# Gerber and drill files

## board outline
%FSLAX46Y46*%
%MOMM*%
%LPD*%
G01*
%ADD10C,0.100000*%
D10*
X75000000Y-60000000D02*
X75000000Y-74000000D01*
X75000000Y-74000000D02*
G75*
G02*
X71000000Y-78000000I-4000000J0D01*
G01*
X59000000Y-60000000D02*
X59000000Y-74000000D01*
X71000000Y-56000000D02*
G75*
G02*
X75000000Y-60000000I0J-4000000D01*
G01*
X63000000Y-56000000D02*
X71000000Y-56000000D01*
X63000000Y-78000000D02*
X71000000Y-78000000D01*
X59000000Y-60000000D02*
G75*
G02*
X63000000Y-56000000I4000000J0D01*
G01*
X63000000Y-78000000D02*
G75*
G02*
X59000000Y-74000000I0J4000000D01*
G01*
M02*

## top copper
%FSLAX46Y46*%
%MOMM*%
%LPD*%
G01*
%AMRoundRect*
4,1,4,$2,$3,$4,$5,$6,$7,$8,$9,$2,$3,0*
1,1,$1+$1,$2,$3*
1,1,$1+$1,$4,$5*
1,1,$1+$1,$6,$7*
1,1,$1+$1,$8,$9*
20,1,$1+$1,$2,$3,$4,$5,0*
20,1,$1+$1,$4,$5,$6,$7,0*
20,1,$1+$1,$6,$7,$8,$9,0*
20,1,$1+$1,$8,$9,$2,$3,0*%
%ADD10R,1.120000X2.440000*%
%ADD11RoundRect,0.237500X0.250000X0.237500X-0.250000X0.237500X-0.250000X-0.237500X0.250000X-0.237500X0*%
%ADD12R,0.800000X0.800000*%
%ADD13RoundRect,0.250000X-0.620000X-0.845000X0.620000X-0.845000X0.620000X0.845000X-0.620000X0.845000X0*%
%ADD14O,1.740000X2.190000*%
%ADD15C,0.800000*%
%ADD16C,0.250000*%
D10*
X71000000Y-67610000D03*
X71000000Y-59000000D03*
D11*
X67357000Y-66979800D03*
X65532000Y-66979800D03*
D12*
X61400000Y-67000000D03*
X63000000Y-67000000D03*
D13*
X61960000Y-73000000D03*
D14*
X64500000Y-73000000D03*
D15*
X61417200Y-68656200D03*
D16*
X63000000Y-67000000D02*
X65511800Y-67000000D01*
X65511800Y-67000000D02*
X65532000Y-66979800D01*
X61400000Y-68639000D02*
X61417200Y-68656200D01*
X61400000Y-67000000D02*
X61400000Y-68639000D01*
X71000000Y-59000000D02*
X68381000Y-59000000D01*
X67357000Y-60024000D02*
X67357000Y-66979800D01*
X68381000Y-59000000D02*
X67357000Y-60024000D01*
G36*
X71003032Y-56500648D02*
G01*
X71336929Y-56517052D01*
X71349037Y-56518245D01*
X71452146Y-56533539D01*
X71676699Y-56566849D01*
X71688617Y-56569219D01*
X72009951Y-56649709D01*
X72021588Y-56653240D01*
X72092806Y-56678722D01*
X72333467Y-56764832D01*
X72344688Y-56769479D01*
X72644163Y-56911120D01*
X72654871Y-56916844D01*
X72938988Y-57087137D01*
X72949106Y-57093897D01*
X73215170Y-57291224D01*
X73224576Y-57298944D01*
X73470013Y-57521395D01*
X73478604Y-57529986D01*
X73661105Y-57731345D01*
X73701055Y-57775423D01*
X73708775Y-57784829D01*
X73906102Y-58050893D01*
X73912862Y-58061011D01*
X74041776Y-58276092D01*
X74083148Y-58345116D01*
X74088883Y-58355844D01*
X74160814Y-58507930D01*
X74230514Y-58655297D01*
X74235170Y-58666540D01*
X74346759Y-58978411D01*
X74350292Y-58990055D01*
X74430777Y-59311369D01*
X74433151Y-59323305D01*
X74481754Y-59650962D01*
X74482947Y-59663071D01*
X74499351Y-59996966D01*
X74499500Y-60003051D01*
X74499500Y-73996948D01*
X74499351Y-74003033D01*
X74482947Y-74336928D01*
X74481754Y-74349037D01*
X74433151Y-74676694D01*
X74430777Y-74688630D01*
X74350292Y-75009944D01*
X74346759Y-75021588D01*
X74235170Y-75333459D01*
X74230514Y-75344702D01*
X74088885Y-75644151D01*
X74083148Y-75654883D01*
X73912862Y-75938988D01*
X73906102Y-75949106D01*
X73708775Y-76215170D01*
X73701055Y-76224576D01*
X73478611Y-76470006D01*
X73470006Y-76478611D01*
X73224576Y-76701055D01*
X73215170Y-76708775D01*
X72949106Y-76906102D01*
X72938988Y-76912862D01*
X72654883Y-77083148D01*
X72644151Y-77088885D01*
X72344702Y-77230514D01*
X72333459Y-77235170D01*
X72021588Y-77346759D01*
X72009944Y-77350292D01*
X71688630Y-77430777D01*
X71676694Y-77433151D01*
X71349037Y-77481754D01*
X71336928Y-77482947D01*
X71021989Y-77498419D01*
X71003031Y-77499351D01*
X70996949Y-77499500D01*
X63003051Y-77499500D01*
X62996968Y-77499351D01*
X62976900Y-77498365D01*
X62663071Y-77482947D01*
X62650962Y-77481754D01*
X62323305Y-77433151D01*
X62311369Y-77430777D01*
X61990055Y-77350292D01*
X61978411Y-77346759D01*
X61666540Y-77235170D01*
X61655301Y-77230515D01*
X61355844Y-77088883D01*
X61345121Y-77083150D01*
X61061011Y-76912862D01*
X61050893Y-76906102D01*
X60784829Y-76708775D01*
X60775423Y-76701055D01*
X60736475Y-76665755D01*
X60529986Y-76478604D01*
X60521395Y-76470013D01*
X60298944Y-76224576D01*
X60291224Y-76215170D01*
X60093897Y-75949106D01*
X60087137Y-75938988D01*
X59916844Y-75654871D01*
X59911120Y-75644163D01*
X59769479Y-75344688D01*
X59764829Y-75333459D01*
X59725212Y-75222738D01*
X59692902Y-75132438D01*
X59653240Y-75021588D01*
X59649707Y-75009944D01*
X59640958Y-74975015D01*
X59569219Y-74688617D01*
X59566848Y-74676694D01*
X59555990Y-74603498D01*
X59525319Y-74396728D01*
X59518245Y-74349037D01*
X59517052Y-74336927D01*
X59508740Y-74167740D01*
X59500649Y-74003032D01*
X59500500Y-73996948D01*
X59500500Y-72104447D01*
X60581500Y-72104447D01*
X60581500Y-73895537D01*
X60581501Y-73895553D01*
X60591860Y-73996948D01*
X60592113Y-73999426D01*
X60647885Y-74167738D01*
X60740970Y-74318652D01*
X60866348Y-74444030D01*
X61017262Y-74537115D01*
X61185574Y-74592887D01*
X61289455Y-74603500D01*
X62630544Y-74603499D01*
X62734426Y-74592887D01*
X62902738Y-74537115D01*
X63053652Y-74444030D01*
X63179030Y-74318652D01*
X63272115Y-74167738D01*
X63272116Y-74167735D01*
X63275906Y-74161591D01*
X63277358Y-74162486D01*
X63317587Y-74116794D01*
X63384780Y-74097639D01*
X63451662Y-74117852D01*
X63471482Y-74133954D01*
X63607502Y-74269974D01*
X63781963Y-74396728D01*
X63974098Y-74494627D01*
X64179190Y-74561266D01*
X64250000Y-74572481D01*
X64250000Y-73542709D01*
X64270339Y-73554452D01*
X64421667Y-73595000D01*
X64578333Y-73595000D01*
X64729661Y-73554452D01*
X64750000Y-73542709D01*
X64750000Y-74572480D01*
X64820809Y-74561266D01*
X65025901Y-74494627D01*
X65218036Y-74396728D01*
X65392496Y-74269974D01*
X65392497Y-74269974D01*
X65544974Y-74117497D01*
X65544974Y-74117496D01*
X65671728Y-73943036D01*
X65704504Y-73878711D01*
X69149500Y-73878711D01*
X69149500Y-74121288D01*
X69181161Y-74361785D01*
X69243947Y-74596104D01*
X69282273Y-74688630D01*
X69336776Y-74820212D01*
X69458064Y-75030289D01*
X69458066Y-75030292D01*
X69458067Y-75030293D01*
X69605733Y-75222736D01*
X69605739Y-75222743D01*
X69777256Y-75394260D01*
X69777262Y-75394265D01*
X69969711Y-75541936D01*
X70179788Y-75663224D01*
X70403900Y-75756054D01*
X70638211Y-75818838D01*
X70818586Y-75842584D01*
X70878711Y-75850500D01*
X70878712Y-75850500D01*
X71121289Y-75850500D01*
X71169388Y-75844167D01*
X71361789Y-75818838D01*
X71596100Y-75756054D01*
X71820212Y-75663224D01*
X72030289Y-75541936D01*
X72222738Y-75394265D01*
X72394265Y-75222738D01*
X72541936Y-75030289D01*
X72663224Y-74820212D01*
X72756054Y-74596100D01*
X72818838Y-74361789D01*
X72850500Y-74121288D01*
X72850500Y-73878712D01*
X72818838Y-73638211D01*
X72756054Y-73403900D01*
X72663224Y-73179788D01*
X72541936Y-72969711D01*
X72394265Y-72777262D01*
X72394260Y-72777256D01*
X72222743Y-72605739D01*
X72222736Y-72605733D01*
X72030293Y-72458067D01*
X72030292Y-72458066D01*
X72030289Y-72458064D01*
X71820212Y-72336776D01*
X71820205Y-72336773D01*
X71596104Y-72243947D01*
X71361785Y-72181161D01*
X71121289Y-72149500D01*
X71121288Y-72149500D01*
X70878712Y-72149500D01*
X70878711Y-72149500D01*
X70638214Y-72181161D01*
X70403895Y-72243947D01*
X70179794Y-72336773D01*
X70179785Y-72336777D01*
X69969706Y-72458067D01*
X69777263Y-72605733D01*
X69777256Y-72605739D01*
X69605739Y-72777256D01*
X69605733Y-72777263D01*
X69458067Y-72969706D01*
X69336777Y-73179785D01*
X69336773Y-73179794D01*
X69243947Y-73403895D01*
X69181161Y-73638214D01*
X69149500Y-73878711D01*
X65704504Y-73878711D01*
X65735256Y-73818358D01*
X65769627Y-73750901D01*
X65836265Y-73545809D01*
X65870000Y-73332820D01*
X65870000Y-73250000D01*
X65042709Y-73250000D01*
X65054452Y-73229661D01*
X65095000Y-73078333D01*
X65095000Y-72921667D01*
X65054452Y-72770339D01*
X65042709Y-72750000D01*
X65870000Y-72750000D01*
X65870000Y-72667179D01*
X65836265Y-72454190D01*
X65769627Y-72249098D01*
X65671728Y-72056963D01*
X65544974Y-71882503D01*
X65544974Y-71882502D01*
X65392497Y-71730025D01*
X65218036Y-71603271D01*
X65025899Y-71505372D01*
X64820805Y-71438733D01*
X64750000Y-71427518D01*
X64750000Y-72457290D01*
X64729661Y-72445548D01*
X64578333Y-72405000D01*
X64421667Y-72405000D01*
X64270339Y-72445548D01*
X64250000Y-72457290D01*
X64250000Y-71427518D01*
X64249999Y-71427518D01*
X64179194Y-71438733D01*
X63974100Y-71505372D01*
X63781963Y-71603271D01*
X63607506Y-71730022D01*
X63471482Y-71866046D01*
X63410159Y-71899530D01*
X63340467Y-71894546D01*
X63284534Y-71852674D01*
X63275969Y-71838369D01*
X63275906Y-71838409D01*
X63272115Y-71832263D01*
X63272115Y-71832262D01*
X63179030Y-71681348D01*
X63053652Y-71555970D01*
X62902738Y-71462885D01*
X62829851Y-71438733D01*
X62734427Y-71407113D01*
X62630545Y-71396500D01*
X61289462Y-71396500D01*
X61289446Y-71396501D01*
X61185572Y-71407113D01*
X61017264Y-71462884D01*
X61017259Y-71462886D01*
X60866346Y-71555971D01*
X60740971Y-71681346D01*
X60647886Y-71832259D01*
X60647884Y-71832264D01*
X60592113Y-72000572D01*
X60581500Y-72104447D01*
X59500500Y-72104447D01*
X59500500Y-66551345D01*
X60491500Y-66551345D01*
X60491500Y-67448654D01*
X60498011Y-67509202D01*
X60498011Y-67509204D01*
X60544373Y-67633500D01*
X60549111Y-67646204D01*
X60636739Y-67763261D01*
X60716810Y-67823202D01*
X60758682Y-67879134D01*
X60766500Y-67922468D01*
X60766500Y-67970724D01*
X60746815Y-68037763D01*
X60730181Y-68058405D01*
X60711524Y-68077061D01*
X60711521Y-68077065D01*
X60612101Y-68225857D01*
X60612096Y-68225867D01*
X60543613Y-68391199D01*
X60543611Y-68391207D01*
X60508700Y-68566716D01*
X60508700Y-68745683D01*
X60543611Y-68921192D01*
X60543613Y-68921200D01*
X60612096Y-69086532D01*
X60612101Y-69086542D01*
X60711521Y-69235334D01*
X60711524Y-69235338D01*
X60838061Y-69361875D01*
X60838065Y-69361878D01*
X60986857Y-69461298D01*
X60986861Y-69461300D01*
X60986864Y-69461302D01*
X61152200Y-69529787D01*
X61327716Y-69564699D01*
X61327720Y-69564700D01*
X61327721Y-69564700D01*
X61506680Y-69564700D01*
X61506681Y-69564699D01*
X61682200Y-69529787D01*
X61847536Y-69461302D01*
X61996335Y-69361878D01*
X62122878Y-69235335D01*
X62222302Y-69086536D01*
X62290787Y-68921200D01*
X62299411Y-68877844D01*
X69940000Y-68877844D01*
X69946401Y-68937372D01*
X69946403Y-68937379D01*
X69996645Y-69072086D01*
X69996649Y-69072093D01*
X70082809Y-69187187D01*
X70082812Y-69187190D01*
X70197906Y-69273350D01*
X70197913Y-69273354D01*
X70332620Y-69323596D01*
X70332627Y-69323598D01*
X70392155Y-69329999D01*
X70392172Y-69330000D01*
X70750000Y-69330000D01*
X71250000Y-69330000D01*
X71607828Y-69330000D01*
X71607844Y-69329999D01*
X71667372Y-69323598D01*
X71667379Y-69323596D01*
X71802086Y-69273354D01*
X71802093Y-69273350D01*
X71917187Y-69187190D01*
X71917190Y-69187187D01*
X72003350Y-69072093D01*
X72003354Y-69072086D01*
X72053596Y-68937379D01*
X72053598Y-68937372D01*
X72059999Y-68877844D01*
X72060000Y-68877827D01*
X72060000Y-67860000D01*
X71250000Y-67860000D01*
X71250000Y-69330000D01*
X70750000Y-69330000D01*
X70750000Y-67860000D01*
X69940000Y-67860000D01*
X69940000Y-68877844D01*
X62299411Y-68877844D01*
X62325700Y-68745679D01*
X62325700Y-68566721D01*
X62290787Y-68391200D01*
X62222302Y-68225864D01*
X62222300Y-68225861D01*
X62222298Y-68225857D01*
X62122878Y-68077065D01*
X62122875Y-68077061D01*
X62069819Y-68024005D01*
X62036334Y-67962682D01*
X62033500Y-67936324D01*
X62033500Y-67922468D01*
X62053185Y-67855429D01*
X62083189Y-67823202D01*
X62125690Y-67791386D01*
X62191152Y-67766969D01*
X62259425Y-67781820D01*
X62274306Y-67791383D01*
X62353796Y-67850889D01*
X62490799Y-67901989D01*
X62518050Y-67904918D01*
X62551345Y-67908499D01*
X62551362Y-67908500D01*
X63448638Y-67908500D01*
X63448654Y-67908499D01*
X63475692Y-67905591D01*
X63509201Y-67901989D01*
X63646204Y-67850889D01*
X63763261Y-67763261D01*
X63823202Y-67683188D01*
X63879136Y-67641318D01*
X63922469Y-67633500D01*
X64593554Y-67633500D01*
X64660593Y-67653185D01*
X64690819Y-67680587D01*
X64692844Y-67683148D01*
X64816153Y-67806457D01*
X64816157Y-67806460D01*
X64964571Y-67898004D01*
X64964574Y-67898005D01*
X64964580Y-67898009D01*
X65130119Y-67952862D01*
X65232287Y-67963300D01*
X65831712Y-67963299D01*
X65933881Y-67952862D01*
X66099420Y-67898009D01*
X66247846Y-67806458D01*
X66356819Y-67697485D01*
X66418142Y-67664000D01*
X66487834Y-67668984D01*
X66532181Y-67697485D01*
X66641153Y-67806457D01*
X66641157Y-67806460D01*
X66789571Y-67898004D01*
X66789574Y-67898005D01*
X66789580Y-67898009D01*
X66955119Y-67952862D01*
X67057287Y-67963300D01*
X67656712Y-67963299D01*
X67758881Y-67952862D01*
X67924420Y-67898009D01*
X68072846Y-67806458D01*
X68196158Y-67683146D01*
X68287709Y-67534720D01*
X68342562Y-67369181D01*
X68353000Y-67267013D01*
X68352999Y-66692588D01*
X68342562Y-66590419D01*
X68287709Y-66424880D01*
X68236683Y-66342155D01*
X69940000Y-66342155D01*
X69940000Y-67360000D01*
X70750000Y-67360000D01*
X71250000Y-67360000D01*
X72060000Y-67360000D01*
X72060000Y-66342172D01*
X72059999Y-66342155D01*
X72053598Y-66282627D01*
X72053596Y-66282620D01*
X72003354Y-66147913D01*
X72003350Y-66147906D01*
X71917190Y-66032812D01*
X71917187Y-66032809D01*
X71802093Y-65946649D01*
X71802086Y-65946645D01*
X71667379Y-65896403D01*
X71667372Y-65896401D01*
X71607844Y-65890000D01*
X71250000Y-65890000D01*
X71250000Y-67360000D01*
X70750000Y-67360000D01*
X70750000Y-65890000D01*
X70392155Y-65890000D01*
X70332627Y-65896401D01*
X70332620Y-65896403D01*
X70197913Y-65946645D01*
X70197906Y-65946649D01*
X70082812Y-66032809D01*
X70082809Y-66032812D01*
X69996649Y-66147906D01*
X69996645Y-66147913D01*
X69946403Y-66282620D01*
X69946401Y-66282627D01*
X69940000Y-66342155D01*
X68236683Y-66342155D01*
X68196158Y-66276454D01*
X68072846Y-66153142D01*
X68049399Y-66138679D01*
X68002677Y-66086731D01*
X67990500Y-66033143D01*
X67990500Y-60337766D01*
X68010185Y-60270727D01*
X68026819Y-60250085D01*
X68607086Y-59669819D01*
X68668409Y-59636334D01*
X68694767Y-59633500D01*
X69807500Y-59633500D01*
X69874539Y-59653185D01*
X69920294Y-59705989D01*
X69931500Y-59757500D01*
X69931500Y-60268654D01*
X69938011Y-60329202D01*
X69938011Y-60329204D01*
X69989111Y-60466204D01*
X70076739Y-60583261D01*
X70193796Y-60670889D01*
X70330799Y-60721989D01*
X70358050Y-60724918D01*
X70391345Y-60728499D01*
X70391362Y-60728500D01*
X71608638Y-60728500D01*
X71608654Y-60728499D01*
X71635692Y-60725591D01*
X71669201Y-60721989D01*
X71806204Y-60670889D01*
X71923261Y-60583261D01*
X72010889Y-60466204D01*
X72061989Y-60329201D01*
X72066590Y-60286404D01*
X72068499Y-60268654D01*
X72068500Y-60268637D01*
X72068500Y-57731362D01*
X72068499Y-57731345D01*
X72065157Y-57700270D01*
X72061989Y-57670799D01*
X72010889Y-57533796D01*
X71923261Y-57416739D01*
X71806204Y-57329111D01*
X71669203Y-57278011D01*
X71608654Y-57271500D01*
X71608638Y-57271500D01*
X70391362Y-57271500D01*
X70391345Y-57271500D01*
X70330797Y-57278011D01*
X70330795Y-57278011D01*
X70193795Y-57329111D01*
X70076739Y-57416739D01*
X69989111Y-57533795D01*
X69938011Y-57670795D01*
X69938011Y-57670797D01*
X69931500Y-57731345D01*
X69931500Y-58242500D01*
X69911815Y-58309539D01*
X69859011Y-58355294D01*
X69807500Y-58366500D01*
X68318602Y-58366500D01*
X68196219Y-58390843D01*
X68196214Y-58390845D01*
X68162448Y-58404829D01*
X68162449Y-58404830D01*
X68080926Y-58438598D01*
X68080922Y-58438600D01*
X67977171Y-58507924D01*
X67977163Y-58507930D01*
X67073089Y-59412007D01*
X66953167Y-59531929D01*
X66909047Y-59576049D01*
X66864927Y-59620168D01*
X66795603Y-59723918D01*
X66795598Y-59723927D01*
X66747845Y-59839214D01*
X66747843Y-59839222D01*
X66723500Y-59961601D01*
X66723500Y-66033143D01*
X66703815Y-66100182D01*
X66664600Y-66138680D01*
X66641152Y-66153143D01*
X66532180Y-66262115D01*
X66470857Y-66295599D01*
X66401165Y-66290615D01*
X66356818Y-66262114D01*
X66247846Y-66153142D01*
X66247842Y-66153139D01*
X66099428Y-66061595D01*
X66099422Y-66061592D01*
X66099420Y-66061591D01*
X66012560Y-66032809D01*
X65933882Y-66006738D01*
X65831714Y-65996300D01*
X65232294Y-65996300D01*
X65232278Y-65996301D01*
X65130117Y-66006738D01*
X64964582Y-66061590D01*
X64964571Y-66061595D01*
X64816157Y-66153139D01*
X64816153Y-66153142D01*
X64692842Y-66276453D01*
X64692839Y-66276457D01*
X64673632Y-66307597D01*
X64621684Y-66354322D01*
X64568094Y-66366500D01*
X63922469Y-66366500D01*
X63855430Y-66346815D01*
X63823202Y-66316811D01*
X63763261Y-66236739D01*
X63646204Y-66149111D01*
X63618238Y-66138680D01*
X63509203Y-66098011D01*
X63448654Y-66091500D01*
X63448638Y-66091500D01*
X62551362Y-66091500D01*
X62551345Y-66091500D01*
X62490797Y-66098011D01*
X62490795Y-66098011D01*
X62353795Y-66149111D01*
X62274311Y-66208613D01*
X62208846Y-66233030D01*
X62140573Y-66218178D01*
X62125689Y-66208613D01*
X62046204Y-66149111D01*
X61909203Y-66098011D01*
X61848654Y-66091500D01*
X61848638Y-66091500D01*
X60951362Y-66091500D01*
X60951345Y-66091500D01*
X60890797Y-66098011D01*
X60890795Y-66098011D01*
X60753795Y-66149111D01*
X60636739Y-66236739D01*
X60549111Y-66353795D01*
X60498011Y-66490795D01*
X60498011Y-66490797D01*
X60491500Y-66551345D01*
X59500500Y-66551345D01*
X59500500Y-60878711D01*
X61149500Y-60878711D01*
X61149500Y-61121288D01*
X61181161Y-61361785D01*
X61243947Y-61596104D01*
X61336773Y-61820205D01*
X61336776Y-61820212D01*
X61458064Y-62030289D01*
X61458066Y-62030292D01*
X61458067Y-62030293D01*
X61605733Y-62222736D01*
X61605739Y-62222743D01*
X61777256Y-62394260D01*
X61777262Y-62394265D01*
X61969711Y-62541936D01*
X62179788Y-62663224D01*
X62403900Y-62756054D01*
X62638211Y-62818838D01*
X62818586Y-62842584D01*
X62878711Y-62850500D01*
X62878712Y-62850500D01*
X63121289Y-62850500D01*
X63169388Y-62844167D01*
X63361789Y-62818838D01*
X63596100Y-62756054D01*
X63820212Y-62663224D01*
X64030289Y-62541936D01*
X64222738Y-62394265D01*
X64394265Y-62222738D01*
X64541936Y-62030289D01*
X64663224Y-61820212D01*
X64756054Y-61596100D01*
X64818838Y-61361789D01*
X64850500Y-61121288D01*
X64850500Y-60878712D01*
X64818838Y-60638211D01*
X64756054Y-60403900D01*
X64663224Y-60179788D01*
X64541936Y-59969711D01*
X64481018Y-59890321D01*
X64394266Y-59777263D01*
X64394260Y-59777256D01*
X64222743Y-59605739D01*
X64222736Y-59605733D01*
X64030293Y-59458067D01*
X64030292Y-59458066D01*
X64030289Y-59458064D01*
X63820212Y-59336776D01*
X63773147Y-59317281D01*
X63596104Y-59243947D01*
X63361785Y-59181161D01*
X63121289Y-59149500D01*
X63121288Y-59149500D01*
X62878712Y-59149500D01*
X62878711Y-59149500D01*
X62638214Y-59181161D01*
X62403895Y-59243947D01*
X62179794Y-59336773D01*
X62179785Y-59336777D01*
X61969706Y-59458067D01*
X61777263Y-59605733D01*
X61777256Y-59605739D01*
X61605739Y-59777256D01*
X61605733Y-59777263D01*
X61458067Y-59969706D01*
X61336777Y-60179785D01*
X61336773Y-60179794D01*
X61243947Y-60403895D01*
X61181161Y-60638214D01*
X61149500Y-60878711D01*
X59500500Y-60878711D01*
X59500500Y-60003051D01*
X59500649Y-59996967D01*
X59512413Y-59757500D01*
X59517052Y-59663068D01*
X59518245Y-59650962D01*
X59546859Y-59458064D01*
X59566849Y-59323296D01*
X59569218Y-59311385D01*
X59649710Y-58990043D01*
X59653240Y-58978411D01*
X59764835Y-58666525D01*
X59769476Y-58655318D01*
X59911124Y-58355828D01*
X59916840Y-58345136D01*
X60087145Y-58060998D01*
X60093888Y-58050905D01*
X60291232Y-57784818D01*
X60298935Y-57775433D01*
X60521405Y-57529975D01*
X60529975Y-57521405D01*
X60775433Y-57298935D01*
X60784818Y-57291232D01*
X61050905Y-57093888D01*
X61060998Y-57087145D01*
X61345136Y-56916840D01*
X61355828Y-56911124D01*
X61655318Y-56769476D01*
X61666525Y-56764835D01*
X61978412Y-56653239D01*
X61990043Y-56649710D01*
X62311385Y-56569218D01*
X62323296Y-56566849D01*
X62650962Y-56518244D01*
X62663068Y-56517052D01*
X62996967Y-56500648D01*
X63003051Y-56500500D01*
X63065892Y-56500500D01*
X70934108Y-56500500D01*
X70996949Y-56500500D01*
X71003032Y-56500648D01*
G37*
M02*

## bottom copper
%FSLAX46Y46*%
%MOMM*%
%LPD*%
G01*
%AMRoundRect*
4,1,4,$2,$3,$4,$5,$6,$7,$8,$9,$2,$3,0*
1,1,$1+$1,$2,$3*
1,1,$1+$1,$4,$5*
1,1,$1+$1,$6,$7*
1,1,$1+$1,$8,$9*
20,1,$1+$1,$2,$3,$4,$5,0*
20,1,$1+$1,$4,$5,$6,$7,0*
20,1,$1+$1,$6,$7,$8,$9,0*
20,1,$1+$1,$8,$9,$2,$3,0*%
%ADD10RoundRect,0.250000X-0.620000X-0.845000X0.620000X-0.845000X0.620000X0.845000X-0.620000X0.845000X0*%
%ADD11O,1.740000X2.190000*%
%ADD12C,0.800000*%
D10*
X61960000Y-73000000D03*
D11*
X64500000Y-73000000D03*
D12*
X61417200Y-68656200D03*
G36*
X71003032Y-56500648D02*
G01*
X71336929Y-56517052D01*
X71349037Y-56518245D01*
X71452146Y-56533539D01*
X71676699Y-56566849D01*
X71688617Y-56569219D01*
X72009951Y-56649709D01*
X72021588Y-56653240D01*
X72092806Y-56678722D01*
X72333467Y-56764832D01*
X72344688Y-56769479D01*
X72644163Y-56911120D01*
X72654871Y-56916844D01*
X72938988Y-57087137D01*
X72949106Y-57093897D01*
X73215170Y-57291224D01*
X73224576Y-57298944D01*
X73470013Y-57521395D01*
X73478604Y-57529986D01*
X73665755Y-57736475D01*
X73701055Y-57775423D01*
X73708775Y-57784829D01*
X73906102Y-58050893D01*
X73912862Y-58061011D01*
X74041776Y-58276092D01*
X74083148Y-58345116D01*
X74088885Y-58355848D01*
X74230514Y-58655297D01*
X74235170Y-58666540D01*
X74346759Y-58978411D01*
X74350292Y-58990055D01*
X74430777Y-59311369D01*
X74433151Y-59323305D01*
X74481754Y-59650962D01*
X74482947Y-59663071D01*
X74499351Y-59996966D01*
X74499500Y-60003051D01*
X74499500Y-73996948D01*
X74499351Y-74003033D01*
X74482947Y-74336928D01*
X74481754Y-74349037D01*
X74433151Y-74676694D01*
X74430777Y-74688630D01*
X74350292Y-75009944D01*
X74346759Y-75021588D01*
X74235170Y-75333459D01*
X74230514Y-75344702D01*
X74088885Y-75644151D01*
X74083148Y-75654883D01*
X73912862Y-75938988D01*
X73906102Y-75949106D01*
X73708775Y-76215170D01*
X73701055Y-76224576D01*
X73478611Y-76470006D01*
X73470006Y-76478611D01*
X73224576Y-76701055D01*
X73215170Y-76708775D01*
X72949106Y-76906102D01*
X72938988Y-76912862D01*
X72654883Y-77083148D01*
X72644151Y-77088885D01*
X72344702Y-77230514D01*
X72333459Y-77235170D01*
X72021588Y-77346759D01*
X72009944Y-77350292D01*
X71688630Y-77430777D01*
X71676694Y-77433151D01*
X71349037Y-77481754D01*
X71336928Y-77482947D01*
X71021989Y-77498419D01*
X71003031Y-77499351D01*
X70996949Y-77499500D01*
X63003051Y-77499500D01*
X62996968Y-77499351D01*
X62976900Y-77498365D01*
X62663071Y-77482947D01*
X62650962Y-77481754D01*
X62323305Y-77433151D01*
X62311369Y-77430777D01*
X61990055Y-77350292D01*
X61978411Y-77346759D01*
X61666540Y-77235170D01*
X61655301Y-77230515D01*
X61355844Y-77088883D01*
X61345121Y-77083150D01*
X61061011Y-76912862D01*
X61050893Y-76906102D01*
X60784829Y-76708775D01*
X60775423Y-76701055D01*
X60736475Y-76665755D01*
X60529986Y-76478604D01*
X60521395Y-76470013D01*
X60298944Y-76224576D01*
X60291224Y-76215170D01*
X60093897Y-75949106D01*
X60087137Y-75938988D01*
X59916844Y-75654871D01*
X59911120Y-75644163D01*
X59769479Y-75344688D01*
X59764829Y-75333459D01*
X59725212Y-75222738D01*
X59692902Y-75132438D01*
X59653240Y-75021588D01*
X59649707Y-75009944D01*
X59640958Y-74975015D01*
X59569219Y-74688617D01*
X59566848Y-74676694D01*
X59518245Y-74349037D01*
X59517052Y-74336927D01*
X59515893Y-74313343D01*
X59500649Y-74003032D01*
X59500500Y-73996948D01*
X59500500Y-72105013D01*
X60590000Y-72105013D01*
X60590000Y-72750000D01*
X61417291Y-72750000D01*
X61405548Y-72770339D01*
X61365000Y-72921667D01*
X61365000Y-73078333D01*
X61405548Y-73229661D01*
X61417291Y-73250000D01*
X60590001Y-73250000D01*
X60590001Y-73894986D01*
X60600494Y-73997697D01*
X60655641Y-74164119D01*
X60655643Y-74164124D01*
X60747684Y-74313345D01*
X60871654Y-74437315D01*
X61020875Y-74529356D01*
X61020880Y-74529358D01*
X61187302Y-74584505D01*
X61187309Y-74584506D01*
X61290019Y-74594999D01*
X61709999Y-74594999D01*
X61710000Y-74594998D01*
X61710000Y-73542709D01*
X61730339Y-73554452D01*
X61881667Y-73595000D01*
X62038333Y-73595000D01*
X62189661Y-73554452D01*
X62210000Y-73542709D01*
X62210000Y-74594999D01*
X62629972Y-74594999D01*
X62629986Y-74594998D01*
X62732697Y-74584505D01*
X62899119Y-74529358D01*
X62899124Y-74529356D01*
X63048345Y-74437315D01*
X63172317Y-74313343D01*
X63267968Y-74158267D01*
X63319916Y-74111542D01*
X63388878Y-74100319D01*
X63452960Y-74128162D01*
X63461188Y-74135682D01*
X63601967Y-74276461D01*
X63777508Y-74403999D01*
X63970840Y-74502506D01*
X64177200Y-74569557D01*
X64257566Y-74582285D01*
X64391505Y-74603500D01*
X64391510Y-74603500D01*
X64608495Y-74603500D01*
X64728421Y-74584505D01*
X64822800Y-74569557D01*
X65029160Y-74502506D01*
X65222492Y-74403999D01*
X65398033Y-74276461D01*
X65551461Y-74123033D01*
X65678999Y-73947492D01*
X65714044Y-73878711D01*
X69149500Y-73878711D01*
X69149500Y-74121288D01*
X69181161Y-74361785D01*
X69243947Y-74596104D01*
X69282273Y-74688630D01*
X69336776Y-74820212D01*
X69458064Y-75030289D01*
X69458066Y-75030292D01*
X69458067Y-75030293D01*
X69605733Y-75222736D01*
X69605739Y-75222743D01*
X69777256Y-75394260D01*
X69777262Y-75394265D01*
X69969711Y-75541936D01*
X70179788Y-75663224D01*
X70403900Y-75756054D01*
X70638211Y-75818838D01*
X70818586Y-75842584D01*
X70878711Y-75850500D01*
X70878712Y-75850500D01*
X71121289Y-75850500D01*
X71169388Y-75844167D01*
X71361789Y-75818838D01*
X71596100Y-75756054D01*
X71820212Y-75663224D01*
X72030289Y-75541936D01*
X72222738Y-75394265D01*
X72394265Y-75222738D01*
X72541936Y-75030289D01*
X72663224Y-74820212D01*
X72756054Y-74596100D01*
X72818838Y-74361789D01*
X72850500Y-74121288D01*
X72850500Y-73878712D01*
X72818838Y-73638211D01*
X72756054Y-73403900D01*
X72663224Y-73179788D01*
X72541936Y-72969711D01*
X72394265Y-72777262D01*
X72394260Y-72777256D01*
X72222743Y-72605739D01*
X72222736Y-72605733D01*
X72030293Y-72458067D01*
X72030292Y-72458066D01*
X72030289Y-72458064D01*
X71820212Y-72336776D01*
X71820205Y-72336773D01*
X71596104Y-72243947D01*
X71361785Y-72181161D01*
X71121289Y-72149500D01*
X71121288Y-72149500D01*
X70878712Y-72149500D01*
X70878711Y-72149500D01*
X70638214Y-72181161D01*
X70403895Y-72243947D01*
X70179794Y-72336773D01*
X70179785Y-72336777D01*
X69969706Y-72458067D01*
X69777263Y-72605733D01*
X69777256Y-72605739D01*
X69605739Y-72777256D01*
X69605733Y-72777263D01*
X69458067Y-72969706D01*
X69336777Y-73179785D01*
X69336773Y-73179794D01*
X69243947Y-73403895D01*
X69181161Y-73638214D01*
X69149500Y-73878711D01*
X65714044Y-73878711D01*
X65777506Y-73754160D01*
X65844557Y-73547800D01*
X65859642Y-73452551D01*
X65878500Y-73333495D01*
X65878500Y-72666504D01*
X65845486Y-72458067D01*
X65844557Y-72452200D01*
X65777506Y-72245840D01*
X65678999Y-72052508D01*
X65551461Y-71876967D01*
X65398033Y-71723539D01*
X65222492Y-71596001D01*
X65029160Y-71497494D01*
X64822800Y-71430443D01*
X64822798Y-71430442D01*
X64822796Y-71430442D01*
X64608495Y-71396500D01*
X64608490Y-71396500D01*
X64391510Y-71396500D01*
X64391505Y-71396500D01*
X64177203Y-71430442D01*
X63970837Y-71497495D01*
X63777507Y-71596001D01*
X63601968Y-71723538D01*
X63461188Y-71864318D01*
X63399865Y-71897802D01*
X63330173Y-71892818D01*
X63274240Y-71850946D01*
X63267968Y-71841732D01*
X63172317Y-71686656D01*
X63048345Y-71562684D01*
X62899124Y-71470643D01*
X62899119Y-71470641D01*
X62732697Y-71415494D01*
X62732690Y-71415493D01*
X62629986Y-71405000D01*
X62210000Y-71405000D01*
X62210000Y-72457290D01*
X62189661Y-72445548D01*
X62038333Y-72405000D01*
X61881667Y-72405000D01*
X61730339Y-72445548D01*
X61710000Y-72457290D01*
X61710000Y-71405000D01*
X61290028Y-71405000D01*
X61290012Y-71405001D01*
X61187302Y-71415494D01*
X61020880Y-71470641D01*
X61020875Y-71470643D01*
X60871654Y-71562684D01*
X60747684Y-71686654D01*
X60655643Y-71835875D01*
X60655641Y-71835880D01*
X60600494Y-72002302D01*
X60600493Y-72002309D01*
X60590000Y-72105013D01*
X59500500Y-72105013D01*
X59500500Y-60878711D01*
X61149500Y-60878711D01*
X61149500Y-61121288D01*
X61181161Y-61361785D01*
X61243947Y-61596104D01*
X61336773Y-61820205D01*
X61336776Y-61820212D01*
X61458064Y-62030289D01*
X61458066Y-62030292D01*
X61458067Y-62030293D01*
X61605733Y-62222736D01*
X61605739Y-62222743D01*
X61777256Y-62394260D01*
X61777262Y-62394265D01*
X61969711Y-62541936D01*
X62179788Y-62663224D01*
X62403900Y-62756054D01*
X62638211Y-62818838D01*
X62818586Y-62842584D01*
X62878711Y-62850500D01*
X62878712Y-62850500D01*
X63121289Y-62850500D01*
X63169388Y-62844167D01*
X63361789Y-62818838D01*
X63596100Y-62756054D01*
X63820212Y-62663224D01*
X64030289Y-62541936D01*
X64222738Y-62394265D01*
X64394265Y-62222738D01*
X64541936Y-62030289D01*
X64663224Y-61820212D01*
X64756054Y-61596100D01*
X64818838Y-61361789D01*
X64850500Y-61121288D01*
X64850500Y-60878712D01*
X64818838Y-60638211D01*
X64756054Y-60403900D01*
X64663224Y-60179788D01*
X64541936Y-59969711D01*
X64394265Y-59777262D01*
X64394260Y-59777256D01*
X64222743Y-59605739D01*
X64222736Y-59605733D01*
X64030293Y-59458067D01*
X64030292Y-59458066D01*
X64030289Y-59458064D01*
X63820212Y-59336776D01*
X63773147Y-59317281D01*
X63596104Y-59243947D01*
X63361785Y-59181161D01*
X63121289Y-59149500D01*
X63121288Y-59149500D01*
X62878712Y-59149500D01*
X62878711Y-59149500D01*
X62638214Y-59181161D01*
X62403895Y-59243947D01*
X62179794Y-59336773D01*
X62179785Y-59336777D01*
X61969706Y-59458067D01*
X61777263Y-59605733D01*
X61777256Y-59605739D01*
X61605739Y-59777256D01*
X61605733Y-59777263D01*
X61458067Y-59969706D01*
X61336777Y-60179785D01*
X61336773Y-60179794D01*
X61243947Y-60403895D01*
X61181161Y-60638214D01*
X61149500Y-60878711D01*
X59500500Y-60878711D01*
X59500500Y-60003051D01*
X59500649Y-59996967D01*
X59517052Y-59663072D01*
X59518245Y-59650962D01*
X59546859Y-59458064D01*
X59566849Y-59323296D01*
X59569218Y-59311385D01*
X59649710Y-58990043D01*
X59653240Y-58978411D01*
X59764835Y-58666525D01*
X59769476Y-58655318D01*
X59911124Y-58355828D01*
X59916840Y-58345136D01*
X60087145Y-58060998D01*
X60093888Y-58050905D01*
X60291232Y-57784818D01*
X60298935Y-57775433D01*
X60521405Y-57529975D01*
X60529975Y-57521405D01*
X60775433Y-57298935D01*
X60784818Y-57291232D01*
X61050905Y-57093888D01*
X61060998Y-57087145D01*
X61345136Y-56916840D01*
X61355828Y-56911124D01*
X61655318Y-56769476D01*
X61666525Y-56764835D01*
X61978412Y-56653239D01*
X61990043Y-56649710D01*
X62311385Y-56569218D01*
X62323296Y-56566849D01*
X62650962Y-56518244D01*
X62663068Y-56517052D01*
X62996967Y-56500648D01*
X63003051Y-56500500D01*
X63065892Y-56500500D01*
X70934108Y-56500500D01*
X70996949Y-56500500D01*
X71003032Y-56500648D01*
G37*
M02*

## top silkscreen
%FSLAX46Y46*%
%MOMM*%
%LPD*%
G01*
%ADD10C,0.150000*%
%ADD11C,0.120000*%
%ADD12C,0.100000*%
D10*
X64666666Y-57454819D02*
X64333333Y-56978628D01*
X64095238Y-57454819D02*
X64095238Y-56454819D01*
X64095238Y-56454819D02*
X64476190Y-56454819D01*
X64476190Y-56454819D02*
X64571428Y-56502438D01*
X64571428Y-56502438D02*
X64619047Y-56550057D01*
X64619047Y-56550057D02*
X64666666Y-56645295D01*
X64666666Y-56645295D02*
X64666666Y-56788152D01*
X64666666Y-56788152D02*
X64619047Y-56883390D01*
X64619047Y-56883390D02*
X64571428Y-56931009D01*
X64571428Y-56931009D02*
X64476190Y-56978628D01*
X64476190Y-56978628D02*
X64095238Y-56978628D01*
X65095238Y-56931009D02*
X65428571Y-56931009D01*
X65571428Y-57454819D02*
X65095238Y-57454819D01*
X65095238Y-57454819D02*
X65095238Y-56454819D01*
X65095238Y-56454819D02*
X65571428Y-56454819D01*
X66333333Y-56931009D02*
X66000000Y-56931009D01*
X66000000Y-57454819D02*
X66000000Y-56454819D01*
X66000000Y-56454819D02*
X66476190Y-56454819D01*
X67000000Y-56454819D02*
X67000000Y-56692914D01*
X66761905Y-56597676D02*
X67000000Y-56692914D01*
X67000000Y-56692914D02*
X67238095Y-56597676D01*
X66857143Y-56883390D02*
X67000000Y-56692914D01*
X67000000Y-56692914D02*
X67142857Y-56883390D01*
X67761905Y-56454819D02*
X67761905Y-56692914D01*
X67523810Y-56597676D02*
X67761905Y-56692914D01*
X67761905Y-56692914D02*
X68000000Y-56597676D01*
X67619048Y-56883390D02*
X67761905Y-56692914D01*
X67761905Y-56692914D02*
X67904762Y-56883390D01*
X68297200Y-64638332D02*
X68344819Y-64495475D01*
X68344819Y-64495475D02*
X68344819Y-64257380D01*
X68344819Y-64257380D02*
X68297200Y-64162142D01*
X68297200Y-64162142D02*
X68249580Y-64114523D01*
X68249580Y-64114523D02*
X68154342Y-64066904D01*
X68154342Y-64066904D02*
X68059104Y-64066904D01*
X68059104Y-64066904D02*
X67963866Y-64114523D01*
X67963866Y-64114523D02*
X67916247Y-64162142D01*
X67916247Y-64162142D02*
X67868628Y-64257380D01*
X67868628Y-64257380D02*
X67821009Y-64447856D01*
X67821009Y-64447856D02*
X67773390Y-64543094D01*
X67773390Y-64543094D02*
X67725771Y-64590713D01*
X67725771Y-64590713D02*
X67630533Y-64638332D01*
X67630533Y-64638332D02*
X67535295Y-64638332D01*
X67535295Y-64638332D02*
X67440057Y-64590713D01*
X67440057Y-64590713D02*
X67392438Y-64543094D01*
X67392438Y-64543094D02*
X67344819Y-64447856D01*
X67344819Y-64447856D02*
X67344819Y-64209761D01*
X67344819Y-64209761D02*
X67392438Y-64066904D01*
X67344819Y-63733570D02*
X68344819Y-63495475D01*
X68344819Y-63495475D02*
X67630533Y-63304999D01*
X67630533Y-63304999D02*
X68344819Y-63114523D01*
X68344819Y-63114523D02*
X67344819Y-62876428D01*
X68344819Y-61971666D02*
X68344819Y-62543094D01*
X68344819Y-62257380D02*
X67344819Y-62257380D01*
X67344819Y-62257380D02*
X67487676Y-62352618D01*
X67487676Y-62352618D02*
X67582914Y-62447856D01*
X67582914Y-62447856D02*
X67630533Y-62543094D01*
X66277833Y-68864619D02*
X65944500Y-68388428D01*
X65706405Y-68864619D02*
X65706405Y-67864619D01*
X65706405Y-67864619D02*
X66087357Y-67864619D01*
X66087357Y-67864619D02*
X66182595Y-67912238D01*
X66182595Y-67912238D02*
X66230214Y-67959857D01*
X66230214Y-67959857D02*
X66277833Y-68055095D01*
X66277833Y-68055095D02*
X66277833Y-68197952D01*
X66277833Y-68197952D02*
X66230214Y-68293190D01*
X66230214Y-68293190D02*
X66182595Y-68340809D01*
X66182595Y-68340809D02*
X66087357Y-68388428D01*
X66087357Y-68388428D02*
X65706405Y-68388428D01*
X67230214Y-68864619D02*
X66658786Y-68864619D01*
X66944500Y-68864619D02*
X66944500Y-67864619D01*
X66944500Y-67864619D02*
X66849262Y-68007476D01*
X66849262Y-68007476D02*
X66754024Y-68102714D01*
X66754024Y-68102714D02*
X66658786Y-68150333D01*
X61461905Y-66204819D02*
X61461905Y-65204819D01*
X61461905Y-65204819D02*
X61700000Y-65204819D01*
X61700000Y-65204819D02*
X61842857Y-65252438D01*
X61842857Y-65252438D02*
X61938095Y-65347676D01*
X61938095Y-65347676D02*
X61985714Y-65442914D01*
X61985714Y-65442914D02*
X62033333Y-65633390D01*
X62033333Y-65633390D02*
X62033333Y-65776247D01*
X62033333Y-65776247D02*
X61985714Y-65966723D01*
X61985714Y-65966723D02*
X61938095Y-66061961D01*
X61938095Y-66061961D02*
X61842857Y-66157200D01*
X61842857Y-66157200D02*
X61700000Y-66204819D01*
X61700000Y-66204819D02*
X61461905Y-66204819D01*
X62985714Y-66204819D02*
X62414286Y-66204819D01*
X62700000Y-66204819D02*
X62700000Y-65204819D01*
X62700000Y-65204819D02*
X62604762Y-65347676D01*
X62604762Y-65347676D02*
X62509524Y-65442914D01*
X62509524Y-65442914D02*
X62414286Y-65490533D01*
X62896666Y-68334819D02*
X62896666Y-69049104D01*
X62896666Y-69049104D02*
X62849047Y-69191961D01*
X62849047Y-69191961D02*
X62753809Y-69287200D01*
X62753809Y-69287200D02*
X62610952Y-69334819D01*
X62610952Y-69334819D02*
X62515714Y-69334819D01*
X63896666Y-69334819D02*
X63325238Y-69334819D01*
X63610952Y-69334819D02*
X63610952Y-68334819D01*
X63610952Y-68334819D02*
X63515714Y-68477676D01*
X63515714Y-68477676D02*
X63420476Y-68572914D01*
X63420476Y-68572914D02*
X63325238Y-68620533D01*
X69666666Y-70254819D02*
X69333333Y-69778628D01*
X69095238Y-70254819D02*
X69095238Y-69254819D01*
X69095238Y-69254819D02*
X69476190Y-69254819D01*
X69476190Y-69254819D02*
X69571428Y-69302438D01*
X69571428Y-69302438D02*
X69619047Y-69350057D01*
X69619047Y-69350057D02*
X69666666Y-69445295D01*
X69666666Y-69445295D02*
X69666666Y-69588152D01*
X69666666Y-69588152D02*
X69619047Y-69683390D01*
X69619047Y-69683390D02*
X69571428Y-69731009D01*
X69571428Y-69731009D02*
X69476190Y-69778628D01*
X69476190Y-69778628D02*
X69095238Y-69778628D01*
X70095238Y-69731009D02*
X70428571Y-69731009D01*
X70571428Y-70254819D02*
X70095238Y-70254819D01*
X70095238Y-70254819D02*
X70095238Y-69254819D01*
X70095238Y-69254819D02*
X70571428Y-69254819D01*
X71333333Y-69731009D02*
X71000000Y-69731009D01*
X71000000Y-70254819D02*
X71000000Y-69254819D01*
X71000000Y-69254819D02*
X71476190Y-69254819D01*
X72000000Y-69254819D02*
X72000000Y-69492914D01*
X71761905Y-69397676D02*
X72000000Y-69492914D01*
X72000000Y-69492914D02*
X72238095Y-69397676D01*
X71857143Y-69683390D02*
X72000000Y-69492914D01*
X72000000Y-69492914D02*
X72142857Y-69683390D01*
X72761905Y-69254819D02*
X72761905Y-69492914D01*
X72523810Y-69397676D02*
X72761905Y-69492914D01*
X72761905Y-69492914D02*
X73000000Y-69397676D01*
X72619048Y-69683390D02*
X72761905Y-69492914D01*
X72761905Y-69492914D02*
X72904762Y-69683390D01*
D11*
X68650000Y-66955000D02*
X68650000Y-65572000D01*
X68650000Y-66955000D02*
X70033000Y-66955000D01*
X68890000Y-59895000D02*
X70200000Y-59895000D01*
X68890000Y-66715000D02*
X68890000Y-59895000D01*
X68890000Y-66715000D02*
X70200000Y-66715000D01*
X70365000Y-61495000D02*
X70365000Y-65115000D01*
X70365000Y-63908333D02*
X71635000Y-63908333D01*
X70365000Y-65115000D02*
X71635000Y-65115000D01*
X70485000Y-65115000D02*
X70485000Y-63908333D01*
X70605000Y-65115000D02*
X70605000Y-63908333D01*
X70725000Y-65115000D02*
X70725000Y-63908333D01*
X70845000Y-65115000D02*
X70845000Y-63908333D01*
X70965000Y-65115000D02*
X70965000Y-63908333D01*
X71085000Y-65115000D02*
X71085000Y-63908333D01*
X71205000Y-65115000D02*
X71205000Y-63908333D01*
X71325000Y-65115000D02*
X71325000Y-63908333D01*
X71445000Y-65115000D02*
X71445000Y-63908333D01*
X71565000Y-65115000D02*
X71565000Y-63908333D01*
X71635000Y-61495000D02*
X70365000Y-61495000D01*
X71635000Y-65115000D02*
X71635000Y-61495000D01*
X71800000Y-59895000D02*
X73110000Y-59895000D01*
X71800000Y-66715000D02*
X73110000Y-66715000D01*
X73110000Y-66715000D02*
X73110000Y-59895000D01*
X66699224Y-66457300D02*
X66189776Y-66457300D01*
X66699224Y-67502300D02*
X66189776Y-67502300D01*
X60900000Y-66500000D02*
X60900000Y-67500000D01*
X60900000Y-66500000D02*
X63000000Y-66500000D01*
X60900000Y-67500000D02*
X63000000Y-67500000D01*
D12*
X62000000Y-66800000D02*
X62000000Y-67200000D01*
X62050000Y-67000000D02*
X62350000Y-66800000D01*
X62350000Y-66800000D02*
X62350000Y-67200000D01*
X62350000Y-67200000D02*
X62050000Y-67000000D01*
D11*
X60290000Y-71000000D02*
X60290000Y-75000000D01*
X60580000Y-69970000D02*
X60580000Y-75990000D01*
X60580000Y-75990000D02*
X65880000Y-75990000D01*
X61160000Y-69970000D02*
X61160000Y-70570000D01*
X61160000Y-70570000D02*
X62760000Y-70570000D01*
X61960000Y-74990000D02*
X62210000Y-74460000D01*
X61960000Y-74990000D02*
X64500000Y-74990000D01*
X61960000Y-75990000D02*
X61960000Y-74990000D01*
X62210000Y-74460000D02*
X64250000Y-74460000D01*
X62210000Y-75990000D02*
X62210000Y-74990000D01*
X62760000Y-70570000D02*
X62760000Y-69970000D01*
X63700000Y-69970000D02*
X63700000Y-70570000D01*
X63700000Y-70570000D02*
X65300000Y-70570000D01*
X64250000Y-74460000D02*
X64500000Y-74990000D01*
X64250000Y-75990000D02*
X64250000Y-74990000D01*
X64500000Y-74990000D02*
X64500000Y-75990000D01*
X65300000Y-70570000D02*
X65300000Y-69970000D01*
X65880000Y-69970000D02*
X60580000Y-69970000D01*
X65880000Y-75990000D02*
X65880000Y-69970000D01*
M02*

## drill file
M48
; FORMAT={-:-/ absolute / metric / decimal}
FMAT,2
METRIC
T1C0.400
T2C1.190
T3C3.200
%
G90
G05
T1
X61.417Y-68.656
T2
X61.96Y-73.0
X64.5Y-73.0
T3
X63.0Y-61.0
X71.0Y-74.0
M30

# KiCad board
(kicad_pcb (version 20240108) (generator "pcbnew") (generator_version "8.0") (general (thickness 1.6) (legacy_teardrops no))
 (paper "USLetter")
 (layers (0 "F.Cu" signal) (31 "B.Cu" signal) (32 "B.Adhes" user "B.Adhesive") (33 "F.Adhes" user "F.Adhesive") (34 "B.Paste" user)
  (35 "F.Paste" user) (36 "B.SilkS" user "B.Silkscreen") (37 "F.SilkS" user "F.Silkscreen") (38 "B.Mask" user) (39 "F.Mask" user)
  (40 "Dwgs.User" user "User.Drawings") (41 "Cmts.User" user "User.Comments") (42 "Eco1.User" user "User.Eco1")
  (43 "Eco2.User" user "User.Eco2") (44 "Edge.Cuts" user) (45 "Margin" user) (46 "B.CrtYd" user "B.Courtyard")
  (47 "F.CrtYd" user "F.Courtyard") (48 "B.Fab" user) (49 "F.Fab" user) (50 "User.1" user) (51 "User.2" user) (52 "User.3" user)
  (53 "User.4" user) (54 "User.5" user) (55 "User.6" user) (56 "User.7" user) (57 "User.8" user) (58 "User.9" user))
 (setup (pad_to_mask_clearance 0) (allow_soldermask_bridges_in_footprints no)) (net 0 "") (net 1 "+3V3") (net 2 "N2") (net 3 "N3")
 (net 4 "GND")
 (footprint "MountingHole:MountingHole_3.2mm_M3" (layer "F.Cu") (at 63 61)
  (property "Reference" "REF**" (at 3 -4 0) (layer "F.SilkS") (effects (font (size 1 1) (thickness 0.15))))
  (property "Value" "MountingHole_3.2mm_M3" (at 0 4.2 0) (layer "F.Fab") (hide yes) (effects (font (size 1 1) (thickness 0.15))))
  (pad "" np_thru_hole circle (at 0 0) (size 3.2 3.2) (drill 3.2) (layers "*.Cu" "*.Mask")))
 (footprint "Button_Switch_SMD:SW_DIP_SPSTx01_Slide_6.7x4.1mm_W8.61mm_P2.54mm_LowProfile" (layer "F.Cu") (at 71 63.305 90)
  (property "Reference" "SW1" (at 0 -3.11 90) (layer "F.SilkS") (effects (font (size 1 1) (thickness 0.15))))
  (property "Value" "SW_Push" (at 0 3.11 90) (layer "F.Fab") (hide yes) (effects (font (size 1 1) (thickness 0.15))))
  (fp_line (start -3.65 -2.35) (end -2.267 -2.35) (stroke (width 0.12) (type solid)) (layer "F.SilkS"))
  (fp_line (start -3.65 -2.35) (end -3.65 -0.967) (stroke (width 0.12) (type solid)) (layer "F.SilkS"))
  (fp_line (start 3.41 -2.11) (end 3.41 -0.8) (stroke (width 0.12) (type solid)) (layer "F.SilkS"))
  (fp_line (start -3.41 -2.11) (end 3.41 -2.11) (stroke (width 0.12) (type solid)) (layer "F.SilkS"))
  (fp_line (start -3.41 -2.11) (end -3.41 -0.8) (stroke (width 0.12) (type solid)) (layer "F.SilkS"))
  (fp_line (start 1.81 -0.635) (end -1.81 -0.635) (stroke (width 0.12) (type solid)) (layer "F.SilkS"))
  (fp_line (start -0.603333 -0.635) (end -0.603333 0.635) (stroke (width 0.12) (type solid)) (layer "F.SilkS"))
  (fp_line (start -1.81 -0.635) (end -1.81 0.635) (stroke (width 0.12) (type solid)) (layer "F.SilkS"))
  (fp_line (start -1.81 -0.515) (end -0.603333 -0.515) (stroke (width 0.12) (type solid)) (layer "F.SilkS"))
  (fp_line (start -1.81 -0.395) (end -0.603333 -0.395) (stroke (width 0.12) (type solid)) (layer "F.SilkS"))
  (fp_line (start -1.81 -0.275) (end -0.603333 -0.275) (stroke (width 0.12) (type solid)) (layer "F.SilkS"))
  (fp_line (start -1.81 -0.155) (end -0.603333 -0.155) (stroke (width 0.12) (type solid)) (layer "F.SilkS"))
  (fp_line (start -1.81 -0.035) (end -0.603333 -0.035) (stroke (width 0.12) (type solid)) (layer "F.SilkS"))
  (fp_line (start -1.81 0.085) (end -0.603333 0.085) (stroke (width 0.12) (type solid)) (layer "F.SilkS"))
  (fp_line (start -1.81 0.205) (end -0.603333 0.205) (stroke (width 0.12) (type solid)) (layer "F.SilkS"))
  (fp_line (start -1.81 0.325) (end -0.603333 0.325) (stroke (width 0.12) (type solid)) (layer "F.SilkS"))
  (fp_line (start -1.81 0.445) (end -0.603333 0.445) (stroke (width 0.12) (type solid)) (layer "F.SilkS"))
  (fp_line (start -1.81 0.565) (end -0.603333 0.565) (stroke (width 0.12) (type solid)) (layer "F.SilkS"))
  (fp_line (start 1.81 0.635) (end 1.81 -0.635) (stroke (width 0.12) (type solid)) (layer "F.SilkS"))
  (fp_line (start -1.81 0.635) (end 1.81 0.635) (stroke (width 0.12) (type solid)) (layer "F.SilkS"))
  (fp_line (start 3.41 0.8) (end 3.41 2.11) (stroke (width 0.12) (type solid)) (layer "F.SilkS"))
  (fp_line (start -3.41 0.8) (end -3.41 2.11) (stroke (width 0.12) (type solid)) (layer "F.SilkS"))
  (fp_line (start -3.41 2.11) (end 3.41 2.11) (stroke (width 0.12) (type solid)) (layer "F.SilkS"))
  (pad "1" smd rect (at -4.305 0 90) (size 2.44 1.12) (layers "F.Cu" "F.Paste" "F.Mask") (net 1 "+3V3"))
  (pad "2" smd rect (at 4.305 0 90) (size 2.44 1.12) (layers "F.Cu" "F.Paste" "F.Mask") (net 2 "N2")))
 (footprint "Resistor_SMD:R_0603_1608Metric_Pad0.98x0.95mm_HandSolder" (layer "F.Cu") (at 66.4445 66.9798 180)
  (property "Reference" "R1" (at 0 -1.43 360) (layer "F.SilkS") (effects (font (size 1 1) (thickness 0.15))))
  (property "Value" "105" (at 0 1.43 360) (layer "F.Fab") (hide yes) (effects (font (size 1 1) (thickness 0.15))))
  (fp_line (start -0.254724 0.5225) (end 0.254724 0.5225) (stroke (width 0.12) (type solid)) (layer "F.SilkS"))
  (fp_line (start -0.254724 -0.5225) (end 0.254724 -0.5225) (stroke (width 0.12) (type solid)) (layer "F.SilkS"))
  (pad "1" smd roundrect (at -0.9125 0 180) (size 0.975 0.95) (layers "F.Cu" "F.Paste" "F.Mask") (roundrect_rratio 0.25) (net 2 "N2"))
  (pad "2" smd roundrect (at 0.9125 0 180) (size 0.975 0.95) (layers "F.Cu" "F.Paste" "F.Mask") (roundrect_rratio 0.25) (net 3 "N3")))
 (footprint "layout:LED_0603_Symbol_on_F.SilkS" (layer "F.Cu") (at 62.2 67)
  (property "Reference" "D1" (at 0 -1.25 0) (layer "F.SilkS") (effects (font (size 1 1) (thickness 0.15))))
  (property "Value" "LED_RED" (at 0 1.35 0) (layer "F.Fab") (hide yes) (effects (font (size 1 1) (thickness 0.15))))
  (fp_line (start -1.3 -0.5) (end -1.3 0.5) (stroke (width 0.12) (type solid)) (layer "F.SilkS"))
  (fp_line (start -1.3 -0.5) (end 0.8 -0.5) (stroke (width 0.12) (type solid)) (layer "F.SilkS"))
  (fp_line (start -1.3 0.5) (end 0.8 0.5) (stroke (width 0.12) (type solid)) (layer "F.SilkS"))
  (fp_line (start -0.2 -0.2) (end -0.2 0.2) (stroke (width 0.1) (type solid)) (layer "F.SilkS"))
  (fp_line (start -0.15 0) (end 0.15 -0.2) (stroke (width 0.1) (type solid)) (layer "F.SilkS"))
  (fp_line (start 0.15 -0.2) (end 0.15 0.2) (stroke (width 0.1) (type solid)) (layer "F.SilkS"))
  (fp_line (start 0.15 0.2) (end -0.15 0) (stroke (width 0.1) (type solid)) (layer "F.SilkS"))
  (pad "1" smd rect (at -0.8 0 180) (size 0.8 0.8) (layers "F.Cu" "F.Paste" "F.Mask") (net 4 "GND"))
  (pad "2" smd rect (at 0.8 0 180) (size 0.8 0.8) (layers "F.Cu" "F.Paste" "F.Mask") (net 3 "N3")))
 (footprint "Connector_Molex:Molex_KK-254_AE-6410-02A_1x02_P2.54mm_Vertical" (layer "F.Cu") (at 61.96 73)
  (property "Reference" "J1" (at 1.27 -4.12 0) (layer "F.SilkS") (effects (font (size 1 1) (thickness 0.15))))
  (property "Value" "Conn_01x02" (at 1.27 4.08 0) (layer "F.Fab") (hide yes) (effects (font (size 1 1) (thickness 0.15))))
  (fp_line (start -1.67 -2) (end -1.67 2) (stroke (width 0.12) (type solid)) (layer "F.SilkS"))
  (fp_line (start -1.38 -3.03) (end -1.38 2.99) (stroke (width 0.12) (type solid)) (layer "F.SilkS"))
  (fp_line (start -1.38 2.99) (end 3.92 2.99) (stroke (width 0.12) (type solid)) (layer "F.SilkS"))
  (fp_line (start -0.8 -3.03) (end -0.8 -2.43) (stroke (width 0.12) (type solid)) (layer "F.SilkS"))
  (fp_line (start -0.8 -2.43) (end 0.8 -2.43) (stroke (width 0.12) (type solid)) (layer "F.SilkS"))
  (fp_line (start 0 1.99) (end 0.25 1.46) (stroke (width 0.12) (type solid)) (layer "F.SilkS"))
  (fp_line (start 0 1.99) (end 2.54 1.99) (stroke (width 0.12) (type solid)) (layer "F.SilkS"))
  (fp_line (start 0 2.99) (end 0 1.99) (stroke (width 0.12) (type solid)) (layer "F.SilkS"))
  (fp_line (start 0.25 1.46) (end 2.29 1.46) (stroke (width 0.12) (type solid)) (layer "F.SilkS"))
  (fp_line (start 0.25 2.99) (end 0.25 1.99) (stroke (width 0.12) (type solid)) (layer "F.SilkS"))
  (fp_line (start 0.8 -2.43) (end 0.8 -3.03) (stroke (width 0.12) (type solid)) (layer "F.SilkS"))
  (fp_line (start 1.74 -3.03) (end 1.74 -2.43) (stroke (width 0.12) (type solid)) (layer "F.SilkS"))
  (fp_line (start 1.74 -2.43) (end 3.34 -2.43) (stroke (width 0.12) (type solid)) (layer "F.SilkS"))
  (fp_line (start 2.29 1.46) (end 2.54 1.99) (stroke (width 0.12) (type solid)) (layer "F.SilkS"))
  (fp_line (start 2.29 2.99) (end 2.29 1.99) (stroke (width 0.12) (type solid)) (layer "F.SilkS"))
  (fp_line (start 2.54 1.99) (end 2.54 2.99) (stroke (width 0.12) (type solid)) (layer "F.SilkS"))
  (fp_line (start 3.34 -2.43) (end 3.34 -3.03) (stroke (width 0.12) (type solid)) (layer "F.SilkS"))
  (fp_line (start 3.92 -3.03) (end -1.38 -3.03) (stroke (width 0.12) (type solid)) (layer "F.SilkS"))
  (fp_line (start 3.92 2.99) (end 3.92 -3.03) (stroke (width 0.12) (type solid)) (layer "F.SilkS"))
  (pad "1" thru_hole roundrect (at 0 0) (size 1.74 2.19) (drill 1.19) (layers "*.Cu" "*.Mask") (remove_unused_layers no)
   (roundrect_rratio 0.143678) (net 4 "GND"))
  (pad "2" thru_hole oval (at 2.54 0) (size 1.74 2.19) (drill 1.19) (layers "*.Cu" "*.Mask") (remove_unused_layers no) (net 1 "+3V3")))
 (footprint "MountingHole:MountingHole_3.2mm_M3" (layer "F.Cu") (at 71 74)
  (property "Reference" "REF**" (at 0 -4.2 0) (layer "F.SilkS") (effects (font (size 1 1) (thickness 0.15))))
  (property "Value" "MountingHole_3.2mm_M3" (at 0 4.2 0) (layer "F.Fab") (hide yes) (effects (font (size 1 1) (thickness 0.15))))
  (pad "" np_thru_hole circle (at 0 0) (size 3.2 3.2) (drill 3.2) (layers "*.Cu" "*.Mask")))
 (gr_line (start 75 60) (end 75 74) (stroke (width 0.1) (type default)) (layer "Edge.Cuts"))
 (gr_arc (start 75 74) (mid 73.828427 76.828427) (end 71 78) (stroke (width 0.1) (type default)) (layer "Edge.Cuts"))
 (gr_line (start 59 60) (end 59 74) (stroke (width 0.1) (type default)) (layer "Edge.Cuts"))
 (gr_arc (start 71 56) (mid 73.828427 57.171573) (end 75 60) (stroke (width 0.1) (type default)) (layer "Edge.Cuts"))
 (gr_line (start 63 56) (end 71 56) (stroke (width 0.1) (type default)) (layer "Edge.Cuts"))
 (gr_line (start 63 78) (end 71 78) (stroke (width 0.1) (type default)) (layer "Edge.Cuts"))
 (gr_arc (start 59 60) (mid 60.171573 57.171573) (end 63 56) (stroke (width 0.1) (type default)) (layer "Edge.Cuts"))
 (gr_arc (start 63 78) (mid 60.171573 76.828427) (end 59 74) (stroke (width 0.1) (type default)) (layer "Edge.Cuts"))
 (segment (start 63 67) (end 65.5118 67) (width 0.25) (layer "F.Cu") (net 3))
 (segment (start 65.5118 67) (end 65.532 66.9798) (width 0.25) (layer "F.Cu") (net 3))
 (segment (start 61.4 68.639) (end 61.4172 68.6562) (width 0.25) (layer "F.Cu") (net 4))
 (segment (start 61.4 67) (end 61.4 68.639) (width 0.25) (layer "F.Cu") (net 4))
 (via (at 61.4172 68.6562) (size 0.8) (drill 0.4) (layers "F.Cu" "B.Cu") (free yes) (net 4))
 (segment (start 71 59) (end 68.381 59) (width 0.25) (layer "F.Cu") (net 2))
 (segment (start 67.357 60.024) (end 67.357 66.9798) (width 0.25) (layer "F.Cu") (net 2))
 (segment (start 68.381 59) (end 67.357 60.024) (width 0.25) (layer "F.Cu") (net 2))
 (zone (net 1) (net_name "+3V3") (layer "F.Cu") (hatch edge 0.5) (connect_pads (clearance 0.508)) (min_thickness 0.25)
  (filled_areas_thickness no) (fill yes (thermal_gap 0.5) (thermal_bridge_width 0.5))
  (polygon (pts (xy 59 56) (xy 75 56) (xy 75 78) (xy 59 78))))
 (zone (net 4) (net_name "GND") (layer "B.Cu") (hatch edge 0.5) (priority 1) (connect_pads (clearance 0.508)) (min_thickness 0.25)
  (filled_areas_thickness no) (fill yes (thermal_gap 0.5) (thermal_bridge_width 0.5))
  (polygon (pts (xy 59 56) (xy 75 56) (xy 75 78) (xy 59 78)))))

